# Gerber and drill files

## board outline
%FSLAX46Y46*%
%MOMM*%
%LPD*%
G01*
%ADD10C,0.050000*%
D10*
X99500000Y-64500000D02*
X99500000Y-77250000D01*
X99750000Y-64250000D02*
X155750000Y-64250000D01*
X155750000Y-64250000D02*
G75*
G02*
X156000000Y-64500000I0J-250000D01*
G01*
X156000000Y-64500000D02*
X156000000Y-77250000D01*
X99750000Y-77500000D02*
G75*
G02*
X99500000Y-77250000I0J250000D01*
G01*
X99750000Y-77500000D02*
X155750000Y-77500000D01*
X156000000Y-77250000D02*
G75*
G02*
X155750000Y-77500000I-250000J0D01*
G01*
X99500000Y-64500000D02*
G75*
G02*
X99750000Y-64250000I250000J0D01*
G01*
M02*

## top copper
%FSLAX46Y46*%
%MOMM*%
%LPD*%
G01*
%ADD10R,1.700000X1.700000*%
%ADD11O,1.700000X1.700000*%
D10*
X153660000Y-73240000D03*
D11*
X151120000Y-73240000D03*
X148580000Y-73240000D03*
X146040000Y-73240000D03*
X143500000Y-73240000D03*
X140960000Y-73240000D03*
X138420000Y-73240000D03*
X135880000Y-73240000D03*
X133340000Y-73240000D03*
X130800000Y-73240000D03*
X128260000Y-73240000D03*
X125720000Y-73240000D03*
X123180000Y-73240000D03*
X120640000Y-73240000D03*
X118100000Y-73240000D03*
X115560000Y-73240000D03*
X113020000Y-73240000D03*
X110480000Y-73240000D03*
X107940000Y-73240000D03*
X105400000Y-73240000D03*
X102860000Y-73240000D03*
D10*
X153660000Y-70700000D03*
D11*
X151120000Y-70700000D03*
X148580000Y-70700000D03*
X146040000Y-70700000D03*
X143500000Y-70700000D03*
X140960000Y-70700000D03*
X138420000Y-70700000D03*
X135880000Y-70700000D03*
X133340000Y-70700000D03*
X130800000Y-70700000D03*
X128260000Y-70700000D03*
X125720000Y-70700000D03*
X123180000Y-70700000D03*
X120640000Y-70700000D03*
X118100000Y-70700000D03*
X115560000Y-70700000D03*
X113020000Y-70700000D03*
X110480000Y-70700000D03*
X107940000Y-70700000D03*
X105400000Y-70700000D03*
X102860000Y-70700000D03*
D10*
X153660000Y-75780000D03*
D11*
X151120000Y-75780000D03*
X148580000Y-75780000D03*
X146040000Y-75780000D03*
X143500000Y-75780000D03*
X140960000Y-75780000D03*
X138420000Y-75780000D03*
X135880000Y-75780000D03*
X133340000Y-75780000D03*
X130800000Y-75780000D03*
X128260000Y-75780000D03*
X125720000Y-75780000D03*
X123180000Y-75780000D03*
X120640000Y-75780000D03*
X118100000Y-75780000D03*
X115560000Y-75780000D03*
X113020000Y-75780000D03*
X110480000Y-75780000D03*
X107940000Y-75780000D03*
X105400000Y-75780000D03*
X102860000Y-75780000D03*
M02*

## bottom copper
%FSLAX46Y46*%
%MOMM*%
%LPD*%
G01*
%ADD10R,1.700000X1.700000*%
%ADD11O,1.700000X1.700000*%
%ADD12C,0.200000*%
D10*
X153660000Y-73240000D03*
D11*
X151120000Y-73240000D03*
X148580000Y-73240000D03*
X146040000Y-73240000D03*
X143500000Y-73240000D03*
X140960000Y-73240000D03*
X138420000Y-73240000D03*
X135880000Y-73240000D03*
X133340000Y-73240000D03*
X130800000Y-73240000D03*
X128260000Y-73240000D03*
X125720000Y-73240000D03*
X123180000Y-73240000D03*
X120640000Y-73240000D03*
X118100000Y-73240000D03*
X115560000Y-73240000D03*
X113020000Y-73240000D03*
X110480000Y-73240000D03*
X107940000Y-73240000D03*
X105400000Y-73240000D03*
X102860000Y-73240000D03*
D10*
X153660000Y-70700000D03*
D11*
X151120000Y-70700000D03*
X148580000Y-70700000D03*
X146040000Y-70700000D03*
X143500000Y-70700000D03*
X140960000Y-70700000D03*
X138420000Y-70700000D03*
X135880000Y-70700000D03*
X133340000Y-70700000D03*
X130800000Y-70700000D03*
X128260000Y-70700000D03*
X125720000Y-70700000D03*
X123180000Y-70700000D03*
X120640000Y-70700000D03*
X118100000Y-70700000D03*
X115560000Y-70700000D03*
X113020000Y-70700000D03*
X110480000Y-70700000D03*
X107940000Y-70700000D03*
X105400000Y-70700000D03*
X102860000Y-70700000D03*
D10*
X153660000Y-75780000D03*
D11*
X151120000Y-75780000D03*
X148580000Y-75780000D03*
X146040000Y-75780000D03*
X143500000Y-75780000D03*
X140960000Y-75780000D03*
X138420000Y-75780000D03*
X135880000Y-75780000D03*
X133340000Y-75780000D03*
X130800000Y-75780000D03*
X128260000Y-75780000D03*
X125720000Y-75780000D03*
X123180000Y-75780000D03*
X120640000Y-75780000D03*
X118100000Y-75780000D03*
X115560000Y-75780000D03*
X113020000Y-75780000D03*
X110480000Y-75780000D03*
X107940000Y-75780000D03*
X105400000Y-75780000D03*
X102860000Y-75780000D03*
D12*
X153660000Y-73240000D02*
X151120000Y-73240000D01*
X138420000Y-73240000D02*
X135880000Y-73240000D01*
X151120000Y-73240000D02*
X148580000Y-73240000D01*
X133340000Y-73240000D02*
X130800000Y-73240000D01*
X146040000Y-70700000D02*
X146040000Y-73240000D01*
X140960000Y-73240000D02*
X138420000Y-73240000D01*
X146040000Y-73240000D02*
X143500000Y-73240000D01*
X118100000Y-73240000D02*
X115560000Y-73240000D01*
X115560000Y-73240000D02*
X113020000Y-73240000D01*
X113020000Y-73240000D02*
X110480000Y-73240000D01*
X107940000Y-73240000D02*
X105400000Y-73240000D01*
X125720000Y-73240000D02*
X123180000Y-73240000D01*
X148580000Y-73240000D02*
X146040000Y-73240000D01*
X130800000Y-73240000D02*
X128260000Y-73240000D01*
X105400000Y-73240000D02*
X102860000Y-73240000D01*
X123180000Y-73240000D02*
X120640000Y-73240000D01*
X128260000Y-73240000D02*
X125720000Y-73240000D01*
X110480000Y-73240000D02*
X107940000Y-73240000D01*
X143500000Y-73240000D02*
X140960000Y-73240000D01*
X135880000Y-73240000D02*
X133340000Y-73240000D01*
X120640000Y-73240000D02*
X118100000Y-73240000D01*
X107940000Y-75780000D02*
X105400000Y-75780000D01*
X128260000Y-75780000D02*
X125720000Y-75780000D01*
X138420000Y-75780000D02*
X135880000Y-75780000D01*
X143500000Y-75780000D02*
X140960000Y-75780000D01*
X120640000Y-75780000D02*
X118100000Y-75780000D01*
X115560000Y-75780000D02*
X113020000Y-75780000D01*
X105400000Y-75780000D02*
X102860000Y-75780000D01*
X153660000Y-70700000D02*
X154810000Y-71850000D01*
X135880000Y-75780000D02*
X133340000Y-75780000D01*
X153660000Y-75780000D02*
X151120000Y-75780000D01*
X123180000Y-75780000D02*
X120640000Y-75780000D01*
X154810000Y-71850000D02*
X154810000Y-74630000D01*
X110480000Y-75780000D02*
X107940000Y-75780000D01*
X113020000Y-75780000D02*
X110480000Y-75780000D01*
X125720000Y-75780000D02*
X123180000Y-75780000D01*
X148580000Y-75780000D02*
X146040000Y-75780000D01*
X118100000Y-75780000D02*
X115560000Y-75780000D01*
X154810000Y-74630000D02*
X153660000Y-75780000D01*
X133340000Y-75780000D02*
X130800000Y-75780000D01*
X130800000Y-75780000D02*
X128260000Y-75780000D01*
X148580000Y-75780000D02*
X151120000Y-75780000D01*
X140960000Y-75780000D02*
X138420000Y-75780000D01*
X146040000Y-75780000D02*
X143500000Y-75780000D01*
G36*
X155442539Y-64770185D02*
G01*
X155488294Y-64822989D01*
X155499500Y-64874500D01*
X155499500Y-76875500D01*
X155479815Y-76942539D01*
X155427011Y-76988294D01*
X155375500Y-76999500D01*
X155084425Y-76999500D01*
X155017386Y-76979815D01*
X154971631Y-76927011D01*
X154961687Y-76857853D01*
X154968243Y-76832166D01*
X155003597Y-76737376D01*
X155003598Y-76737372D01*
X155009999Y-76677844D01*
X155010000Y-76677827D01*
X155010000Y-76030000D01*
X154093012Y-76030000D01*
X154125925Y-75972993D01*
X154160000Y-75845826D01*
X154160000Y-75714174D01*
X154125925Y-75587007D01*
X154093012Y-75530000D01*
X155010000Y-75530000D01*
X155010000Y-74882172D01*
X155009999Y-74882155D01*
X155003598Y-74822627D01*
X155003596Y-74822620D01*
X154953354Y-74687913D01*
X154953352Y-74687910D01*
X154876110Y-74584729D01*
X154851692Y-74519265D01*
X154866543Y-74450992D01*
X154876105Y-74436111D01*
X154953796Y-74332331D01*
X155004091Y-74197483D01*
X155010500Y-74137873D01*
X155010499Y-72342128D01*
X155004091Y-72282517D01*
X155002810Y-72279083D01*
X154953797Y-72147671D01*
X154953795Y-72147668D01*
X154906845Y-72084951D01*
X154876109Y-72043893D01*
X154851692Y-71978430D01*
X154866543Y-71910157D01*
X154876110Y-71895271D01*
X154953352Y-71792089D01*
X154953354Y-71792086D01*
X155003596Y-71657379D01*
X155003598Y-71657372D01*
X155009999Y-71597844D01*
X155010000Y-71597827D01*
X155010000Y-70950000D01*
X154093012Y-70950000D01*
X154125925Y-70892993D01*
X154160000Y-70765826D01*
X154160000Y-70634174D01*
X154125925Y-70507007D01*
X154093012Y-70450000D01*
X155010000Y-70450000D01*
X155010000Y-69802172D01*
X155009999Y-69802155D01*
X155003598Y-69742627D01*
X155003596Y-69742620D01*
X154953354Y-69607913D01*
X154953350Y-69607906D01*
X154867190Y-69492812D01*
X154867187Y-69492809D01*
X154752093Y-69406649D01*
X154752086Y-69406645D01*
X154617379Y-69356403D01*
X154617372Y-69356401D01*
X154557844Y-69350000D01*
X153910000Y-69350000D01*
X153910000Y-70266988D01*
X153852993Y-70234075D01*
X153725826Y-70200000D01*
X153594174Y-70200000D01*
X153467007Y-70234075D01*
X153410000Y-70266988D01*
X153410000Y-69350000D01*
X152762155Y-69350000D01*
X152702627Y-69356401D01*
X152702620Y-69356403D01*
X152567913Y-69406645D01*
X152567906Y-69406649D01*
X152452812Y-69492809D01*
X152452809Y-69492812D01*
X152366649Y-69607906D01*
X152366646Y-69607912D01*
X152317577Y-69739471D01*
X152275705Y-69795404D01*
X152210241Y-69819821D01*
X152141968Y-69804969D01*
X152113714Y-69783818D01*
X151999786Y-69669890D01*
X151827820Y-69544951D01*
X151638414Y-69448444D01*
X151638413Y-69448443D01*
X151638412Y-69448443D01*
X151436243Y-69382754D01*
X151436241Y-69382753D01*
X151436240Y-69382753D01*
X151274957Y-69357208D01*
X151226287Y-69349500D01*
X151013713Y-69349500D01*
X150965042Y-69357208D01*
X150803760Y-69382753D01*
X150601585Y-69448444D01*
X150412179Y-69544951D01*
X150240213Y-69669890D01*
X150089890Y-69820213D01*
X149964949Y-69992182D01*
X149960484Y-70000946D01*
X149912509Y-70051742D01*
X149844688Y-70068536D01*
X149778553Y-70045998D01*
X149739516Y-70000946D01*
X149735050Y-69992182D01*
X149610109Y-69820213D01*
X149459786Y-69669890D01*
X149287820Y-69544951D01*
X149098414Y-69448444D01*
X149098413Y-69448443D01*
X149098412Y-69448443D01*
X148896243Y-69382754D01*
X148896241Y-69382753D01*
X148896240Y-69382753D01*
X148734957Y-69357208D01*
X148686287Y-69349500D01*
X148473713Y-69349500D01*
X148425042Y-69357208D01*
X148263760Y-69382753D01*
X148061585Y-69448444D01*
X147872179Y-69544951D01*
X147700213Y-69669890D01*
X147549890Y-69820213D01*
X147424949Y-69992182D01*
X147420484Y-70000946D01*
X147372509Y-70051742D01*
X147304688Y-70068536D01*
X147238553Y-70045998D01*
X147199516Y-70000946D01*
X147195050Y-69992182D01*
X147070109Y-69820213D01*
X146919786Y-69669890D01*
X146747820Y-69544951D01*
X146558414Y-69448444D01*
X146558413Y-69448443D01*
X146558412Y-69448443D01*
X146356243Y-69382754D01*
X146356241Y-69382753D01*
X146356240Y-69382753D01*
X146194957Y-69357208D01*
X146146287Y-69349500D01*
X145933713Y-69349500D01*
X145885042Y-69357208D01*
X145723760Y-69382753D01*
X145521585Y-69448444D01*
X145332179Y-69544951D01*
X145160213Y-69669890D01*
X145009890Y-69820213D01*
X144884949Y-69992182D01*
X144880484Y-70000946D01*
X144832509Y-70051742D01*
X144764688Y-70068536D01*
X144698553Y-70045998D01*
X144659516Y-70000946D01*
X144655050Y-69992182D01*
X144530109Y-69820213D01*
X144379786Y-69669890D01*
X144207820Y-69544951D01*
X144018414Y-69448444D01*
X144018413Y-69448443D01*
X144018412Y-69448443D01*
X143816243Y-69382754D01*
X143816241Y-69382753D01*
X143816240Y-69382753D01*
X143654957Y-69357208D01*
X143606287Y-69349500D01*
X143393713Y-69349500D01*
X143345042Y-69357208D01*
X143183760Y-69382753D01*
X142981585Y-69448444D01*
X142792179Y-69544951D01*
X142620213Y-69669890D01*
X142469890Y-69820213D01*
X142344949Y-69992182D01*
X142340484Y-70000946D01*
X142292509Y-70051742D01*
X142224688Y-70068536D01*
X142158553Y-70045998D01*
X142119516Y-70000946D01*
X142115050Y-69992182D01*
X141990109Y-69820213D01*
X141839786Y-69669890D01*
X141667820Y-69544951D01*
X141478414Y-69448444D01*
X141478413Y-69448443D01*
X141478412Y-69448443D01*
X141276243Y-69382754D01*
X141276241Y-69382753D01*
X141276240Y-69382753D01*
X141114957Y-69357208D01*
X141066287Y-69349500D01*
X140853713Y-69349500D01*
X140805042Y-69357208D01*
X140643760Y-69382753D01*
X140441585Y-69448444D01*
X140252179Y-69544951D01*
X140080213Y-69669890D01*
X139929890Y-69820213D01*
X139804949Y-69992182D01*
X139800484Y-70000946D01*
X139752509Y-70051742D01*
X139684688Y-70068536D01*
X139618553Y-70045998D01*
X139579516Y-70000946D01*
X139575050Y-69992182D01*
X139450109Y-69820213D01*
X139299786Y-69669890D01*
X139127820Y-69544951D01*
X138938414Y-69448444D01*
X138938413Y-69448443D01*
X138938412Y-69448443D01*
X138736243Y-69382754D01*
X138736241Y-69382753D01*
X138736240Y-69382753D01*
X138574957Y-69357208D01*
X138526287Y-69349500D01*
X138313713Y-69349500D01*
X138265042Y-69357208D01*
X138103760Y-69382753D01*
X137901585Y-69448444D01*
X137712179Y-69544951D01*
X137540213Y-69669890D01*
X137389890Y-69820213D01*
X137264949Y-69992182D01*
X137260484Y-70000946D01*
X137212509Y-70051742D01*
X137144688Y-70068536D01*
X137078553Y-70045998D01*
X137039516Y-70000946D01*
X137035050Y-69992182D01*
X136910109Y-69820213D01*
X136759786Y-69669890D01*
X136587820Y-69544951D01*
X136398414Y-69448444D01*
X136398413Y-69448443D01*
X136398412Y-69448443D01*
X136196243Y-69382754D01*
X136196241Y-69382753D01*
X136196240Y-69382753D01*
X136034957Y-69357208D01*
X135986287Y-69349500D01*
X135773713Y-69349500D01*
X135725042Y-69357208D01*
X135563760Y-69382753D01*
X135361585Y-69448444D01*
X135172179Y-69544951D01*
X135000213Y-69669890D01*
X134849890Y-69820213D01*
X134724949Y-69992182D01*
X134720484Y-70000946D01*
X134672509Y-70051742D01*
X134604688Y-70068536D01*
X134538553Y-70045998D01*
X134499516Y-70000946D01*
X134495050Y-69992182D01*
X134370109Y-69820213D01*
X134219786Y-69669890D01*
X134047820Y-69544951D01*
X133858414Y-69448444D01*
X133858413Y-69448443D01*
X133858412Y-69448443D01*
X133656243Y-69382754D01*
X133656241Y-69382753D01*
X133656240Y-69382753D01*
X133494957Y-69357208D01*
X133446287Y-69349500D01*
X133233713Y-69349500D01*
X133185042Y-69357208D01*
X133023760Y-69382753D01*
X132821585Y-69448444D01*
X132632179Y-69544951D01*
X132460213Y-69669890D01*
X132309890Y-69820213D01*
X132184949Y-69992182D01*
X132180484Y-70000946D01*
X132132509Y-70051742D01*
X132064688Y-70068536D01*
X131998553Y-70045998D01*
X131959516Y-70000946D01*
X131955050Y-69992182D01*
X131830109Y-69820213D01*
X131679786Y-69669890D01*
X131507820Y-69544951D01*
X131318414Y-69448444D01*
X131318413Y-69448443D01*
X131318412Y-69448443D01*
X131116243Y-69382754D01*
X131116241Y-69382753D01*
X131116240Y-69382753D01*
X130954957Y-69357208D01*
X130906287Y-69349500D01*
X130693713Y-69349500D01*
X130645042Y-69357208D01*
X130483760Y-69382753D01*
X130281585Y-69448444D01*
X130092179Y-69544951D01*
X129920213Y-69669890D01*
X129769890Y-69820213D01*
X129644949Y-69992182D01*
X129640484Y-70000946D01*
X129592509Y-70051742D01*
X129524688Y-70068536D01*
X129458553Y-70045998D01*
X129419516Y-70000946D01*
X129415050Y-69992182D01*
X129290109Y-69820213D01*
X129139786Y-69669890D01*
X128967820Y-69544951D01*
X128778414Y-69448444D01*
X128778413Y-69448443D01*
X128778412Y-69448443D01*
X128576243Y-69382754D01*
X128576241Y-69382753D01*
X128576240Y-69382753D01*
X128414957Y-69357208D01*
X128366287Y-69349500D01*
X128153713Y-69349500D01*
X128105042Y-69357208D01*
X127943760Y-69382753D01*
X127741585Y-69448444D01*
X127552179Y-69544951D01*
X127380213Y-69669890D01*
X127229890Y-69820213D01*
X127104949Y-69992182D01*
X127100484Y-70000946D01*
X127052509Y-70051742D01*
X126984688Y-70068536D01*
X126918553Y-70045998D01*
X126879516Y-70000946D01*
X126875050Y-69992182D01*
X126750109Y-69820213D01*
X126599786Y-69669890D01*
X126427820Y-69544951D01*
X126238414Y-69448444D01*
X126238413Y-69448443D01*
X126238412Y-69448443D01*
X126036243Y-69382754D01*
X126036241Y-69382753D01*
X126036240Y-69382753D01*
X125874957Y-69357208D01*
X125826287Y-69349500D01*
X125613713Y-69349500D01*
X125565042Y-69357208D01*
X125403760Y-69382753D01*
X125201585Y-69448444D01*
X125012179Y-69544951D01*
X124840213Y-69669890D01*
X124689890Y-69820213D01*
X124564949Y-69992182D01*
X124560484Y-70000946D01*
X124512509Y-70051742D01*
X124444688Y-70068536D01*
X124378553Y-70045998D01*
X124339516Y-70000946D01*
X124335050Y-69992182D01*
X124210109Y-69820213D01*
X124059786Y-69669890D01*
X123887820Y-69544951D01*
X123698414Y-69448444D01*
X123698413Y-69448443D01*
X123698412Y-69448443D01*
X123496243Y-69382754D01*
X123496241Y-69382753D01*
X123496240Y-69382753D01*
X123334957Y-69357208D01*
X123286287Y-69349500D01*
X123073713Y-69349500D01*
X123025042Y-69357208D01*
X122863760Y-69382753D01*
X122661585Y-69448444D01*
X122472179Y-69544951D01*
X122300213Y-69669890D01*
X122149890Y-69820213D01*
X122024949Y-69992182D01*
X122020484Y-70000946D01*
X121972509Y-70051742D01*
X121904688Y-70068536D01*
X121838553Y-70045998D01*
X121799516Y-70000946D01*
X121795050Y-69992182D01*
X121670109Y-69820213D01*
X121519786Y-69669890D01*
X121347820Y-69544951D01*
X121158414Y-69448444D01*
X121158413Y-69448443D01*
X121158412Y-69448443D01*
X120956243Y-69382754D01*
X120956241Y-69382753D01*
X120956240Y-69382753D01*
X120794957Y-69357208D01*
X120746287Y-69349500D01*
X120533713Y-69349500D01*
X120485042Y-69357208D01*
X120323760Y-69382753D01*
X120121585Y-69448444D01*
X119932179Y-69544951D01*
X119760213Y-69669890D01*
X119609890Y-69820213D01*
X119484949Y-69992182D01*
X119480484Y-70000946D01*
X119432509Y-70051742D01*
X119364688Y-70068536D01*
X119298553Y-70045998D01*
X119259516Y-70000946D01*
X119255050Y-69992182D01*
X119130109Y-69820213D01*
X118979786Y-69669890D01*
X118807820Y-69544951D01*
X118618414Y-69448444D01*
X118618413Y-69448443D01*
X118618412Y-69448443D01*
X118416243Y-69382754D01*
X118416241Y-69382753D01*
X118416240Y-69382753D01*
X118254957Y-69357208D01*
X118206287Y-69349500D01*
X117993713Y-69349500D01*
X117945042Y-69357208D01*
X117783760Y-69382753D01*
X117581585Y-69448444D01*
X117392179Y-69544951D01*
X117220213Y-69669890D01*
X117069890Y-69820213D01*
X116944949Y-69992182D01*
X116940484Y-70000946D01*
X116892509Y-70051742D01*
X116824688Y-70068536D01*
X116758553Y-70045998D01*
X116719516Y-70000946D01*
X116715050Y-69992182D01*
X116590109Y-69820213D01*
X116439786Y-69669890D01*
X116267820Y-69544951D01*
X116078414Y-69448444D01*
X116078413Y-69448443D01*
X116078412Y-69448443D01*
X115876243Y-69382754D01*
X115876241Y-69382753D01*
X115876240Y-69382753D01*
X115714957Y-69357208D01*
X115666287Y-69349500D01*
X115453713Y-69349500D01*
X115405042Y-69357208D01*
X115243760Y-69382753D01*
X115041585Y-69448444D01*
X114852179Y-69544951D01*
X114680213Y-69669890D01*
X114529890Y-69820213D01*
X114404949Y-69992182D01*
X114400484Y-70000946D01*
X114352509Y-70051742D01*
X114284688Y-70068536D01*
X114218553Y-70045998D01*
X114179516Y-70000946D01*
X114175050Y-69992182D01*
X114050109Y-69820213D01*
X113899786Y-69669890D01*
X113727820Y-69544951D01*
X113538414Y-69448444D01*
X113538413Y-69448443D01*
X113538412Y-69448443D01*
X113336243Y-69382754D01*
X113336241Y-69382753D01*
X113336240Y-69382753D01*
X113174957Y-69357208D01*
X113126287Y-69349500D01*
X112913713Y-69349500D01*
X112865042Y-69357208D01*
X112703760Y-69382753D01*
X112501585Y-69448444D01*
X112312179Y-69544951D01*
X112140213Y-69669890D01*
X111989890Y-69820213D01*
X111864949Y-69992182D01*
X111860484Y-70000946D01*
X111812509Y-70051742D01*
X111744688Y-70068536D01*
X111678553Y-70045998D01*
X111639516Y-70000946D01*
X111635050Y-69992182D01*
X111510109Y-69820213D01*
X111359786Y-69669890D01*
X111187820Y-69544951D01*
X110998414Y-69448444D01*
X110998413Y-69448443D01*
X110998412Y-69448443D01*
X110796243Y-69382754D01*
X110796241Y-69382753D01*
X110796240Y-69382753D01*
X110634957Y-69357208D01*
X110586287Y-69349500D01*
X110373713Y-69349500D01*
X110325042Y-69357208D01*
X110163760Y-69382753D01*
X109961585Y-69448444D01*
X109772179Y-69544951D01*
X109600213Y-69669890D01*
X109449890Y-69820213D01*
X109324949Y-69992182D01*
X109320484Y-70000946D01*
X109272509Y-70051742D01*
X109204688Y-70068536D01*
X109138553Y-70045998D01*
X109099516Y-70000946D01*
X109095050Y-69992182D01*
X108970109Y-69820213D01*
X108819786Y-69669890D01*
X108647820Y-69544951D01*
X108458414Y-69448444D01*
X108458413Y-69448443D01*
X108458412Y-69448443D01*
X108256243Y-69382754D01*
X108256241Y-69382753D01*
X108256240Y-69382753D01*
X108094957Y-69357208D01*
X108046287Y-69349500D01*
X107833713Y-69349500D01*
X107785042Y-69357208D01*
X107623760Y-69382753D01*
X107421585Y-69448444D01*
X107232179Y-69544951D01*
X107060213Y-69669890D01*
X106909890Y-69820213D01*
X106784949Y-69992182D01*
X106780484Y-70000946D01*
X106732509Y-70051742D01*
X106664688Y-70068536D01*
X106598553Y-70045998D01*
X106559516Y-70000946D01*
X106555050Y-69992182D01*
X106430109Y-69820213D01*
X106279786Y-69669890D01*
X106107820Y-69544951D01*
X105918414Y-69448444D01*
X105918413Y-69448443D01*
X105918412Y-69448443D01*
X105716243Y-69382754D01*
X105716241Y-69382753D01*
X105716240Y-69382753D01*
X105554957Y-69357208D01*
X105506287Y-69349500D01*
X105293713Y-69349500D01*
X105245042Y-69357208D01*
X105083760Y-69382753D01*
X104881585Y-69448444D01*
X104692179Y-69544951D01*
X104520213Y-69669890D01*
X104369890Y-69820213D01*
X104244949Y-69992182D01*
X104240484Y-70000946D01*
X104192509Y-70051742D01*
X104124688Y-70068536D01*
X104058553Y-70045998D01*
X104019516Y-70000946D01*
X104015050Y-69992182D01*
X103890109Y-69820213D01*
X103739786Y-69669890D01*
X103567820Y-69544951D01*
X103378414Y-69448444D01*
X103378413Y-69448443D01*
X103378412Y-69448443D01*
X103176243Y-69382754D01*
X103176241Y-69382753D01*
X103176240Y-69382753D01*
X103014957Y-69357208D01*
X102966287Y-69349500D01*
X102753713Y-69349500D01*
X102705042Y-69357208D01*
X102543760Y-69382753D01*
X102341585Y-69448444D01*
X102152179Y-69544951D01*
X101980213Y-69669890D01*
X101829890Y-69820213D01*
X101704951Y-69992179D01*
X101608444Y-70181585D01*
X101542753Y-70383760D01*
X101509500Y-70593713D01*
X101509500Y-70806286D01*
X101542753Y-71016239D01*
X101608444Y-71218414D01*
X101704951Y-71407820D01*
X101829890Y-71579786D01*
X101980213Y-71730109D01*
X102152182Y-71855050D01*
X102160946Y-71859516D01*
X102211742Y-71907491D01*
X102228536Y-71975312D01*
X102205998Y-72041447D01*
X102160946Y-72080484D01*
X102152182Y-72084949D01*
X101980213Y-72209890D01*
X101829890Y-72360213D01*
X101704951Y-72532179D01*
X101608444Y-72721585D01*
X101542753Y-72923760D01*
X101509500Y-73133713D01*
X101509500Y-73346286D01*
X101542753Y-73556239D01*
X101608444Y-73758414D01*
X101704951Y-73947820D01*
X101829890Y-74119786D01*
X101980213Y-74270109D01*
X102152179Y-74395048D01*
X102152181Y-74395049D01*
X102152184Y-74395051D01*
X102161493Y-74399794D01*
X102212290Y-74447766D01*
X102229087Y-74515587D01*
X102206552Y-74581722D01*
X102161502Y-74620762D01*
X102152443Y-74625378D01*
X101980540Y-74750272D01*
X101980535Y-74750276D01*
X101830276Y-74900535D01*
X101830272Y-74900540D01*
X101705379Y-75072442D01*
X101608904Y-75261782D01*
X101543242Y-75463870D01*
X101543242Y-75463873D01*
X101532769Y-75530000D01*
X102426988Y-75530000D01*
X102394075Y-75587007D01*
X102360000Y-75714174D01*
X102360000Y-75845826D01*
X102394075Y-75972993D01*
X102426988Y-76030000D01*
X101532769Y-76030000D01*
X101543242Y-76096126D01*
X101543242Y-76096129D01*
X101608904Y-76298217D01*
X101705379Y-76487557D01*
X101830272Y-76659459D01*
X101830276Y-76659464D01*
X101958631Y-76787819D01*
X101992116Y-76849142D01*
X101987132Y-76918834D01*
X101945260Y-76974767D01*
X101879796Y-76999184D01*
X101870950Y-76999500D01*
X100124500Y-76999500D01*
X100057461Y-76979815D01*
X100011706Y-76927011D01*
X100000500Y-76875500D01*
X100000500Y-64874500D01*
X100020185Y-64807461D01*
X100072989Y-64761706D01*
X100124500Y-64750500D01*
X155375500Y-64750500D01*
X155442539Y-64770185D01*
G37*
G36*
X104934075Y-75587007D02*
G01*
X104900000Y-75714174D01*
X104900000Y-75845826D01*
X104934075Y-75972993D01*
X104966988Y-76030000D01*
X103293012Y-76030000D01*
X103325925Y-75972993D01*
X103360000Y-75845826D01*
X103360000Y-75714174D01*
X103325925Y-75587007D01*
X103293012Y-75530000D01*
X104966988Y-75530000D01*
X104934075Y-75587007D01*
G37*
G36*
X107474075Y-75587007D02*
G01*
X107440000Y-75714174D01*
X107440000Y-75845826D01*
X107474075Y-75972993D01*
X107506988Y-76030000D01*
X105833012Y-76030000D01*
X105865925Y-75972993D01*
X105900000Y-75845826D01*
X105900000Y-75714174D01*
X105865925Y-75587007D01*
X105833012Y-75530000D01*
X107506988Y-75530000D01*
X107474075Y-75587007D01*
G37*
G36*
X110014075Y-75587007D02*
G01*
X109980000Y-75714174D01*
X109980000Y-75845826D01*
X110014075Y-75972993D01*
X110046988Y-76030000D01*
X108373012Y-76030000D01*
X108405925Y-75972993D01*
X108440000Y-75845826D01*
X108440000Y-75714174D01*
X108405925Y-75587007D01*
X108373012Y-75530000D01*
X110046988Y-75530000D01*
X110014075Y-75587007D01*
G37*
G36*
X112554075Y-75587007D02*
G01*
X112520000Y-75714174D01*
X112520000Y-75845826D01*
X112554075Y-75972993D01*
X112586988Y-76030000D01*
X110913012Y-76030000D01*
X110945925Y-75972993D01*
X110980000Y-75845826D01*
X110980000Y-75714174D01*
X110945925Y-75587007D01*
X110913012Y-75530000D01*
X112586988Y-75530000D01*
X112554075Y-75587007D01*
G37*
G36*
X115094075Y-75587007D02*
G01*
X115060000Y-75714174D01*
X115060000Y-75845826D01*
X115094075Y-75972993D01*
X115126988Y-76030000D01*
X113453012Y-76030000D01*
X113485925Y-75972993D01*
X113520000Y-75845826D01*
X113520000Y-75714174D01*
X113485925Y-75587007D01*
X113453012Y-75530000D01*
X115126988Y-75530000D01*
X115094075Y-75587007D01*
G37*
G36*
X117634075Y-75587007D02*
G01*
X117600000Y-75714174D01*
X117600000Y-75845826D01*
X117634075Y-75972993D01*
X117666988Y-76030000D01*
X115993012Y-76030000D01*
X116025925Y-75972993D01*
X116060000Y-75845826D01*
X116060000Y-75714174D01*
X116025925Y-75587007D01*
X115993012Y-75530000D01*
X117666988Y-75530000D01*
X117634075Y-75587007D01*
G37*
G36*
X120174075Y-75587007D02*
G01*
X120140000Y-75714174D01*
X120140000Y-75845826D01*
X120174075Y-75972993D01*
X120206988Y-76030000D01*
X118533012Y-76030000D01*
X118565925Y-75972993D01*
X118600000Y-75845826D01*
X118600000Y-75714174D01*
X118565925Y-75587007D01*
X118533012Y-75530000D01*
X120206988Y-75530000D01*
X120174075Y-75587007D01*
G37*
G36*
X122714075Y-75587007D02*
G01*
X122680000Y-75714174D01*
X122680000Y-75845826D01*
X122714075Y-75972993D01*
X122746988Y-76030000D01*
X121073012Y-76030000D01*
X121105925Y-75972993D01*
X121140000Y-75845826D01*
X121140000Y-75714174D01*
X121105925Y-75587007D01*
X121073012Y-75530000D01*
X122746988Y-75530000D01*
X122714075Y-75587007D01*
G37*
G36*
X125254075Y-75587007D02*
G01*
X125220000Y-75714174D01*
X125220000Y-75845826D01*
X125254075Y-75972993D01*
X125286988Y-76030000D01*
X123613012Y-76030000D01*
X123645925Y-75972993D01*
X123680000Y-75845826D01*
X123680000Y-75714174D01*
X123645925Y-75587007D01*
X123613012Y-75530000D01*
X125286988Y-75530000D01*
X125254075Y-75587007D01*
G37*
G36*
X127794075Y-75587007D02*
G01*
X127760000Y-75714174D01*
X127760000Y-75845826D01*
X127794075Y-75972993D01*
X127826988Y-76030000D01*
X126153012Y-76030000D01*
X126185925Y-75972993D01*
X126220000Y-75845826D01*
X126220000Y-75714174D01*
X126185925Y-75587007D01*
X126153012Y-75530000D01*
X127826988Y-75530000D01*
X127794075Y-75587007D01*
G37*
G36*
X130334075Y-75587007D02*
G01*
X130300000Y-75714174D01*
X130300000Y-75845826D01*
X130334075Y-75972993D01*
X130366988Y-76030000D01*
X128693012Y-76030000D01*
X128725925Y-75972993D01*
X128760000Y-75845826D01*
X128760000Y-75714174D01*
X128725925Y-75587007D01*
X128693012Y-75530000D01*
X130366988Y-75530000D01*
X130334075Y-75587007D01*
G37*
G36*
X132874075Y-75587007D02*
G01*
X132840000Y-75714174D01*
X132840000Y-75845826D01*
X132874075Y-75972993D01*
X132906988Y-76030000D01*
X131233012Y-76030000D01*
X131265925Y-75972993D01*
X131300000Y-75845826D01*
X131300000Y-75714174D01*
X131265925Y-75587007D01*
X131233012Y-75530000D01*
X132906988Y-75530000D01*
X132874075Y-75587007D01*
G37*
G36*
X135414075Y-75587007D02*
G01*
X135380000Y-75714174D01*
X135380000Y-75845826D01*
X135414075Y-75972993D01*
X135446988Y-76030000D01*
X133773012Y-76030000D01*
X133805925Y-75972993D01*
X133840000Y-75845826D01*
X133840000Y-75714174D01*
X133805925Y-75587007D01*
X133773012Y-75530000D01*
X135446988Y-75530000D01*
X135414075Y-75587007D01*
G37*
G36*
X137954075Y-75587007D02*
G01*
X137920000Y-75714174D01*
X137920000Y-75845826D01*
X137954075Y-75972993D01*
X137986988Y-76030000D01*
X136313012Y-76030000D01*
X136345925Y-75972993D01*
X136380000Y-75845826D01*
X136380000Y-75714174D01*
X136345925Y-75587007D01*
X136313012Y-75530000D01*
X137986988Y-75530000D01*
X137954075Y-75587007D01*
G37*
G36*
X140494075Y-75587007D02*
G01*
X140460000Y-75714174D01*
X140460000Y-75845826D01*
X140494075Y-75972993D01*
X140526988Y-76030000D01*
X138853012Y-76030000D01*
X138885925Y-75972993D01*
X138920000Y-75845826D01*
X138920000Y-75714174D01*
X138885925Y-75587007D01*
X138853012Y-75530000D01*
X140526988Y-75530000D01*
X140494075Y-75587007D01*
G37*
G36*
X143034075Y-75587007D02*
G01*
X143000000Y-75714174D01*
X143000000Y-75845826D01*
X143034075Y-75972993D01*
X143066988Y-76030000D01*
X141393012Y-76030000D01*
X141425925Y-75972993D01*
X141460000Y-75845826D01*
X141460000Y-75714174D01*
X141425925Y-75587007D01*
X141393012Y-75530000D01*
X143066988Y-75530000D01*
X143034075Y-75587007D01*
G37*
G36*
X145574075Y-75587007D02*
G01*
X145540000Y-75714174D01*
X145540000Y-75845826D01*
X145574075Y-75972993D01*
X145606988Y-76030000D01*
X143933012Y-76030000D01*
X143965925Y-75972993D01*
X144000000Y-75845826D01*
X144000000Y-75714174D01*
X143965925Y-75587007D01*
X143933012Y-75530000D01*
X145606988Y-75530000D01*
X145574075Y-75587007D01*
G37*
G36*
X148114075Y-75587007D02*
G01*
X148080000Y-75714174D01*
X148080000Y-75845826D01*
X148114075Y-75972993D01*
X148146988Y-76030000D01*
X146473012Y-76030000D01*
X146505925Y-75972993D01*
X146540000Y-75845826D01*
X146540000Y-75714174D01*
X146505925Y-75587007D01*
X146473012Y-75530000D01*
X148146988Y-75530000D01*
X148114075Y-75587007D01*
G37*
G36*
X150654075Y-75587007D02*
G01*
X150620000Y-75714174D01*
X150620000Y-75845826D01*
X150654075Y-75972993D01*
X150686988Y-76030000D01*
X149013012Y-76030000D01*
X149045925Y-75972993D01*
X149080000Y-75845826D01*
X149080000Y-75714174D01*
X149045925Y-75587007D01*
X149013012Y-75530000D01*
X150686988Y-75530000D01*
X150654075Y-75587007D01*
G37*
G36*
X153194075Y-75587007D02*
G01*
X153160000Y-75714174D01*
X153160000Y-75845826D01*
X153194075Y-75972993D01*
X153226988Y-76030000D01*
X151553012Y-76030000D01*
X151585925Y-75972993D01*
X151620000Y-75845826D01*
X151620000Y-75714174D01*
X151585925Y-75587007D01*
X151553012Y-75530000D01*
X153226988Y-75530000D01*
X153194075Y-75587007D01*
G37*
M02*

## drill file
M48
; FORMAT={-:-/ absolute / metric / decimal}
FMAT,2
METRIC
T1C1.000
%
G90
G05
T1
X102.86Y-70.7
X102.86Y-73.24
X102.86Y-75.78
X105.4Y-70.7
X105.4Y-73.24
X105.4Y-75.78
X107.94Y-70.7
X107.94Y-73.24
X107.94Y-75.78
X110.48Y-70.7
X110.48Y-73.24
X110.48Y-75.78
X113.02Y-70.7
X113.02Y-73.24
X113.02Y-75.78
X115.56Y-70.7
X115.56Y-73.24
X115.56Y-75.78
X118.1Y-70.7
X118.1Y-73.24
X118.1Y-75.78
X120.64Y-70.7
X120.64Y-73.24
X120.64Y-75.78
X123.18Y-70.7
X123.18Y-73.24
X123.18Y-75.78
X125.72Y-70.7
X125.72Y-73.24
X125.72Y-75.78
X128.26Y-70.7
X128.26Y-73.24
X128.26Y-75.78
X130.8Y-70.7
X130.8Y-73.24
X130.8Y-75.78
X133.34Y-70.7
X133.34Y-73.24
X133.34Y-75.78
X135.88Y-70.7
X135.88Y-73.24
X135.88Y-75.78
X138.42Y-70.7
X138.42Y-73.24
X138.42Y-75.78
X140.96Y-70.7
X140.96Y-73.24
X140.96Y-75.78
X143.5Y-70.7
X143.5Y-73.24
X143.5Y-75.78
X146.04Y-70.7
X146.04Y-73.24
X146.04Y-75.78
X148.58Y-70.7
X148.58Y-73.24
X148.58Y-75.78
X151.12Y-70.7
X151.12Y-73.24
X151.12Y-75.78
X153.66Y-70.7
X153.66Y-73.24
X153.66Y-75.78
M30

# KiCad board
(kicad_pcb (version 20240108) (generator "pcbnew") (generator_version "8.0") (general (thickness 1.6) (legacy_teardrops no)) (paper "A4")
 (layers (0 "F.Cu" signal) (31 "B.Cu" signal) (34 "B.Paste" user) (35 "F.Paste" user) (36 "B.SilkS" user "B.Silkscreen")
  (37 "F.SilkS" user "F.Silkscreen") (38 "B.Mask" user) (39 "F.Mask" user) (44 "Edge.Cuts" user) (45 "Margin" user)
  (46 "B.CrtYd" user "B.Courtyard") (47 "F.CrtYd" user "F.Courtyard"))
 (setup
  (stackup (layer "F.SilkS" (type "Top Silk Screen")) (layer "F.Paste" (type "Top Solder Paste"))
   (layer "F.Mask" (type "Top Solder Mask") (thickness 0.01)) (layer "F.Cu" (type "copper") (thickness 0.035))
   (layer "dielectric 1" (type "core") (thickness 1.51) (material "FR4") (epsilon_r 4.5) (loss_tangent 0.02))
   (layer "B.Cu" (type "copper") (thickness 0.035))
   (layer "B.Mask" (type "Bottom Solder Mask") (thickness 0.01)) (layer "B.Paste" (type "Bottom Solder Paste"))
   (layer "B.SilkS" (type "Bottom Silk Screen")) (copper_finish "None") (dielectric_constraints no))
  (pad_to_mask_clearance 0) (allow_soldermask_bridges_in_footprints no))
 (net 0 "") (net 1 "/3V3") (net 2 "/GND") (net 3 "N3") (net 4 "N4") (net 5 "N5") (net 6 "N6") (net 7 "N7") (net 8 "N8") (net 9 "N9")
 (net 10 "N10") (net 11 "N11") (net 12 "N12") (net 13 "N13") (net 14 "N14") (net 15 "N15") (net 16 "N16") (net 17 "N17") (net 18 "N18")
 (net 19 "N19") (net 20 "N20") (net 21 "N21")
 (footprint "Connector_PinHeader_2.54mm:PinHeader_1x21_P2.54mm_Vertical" (layer "F.Cu") (at 153.66 73.24 -90)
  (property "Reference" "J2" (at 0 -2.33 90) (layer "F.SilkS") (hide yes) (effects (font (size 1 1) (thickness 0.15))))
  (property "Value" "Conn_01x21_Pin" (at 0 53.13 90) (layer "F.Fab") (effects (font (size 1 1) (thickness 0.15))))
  (pad "1" thru_hole rect (at 0 0 270) (size 1.7 1.7) (drill 1) (layers "*.Cu" "*.Mask") (remove_unused_layers no) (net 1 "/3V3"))
  (pad "2" thru_hole oval (at 0 2.54 270) (size 1.7 1.7) (drill 1) (layers "*.Cu" "*.Mask") (remove_unused_layers no) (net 1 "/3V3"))
  (pad "3" thru_hole oval (at 0 5.08 270) (size 1.7 1.7) (drill 1) (layers "*.Cu" "*.Mask") (remove_unused_layers no) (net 1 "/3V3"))
  (pad "4" thru_hole oval (at 0 7.62 270) (size 1.7 1.7) (drill 1) (layers "*.Cu" "*.Mask") (remove_unused_layers no) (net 1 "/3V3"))
  (pad "5" thru_hole oval (at 0 10.16 270) (size 1.7 1.7) (drill 1) (layers "*.Cu" "*.Mask") (remove_unused_layers no) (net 1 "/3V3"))
  (pad "6" thru_hole oval (at 0 12.7 270) (size 1.7 1.7) (drill 1) (layers "*.Cu" "*.Mask") (remove_unused_layers no) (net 1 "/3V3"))
  (pad "7" thru_hole oval (at 0 15.24 270) (size 1.7 1.7) (drill 1) (layers "*.Cu" "*.Mask") (remove_unused_layers no) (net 1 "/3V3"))
  (pad "8" thru_hole oval (at 0 17.78 270) (size 1.7 1.7) (drill 1) (layers "*.Cu" "*.Mask") (remove_unused_layers no) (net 1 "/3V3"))
  (pad "9" thru_hole oval (at 0 20.32 270) (size 1.7 1.7) (drill 1) (layers "*.Cu" "*.Mask") (remove_unused_layers no) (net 1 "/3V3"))
  (pad "10" thru_hole oval (at 0 22.86 270) (size 1.7 1.7) (drill 1) (layers "*.Cu" "*.Mask") (remove_unused_layers no) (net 1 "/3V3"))
  (pad "11" thru_hole oval (at 0 25.4 270) (size 1.7 1.7) (drill 1) (layers "*.Cu" "*.Mask") (remove_unused_layers no) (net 1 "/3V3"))
  (pad "12" thru_hole oval (at 0 27.94 270) (size 1.7 1.7) (drill 1) (layers "*.Cu" "*.Mask") (remove_unused_layers no) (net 1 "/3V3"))
  (pad "13" thru_hole oval (at 0 30.48 270) (size 1.7 1.7) (drill 1) (layers "*.Cu" "*.Mask") (remove_unused_layers no) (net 1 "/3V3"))
  (pad "14" thru_hole oval (at 0 33.02 270) (size 1.7 1.7) (drill 1) (layers "*.Cu" "*.Mask") (remove_unused_layers no) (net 1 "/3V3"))
  (pad "15" thru_hole oval (at 0 35.56 270) (size 1.7 1.7) (drill 1) (layers "*.Cu" "*.Mask") (remove_unused_layers no) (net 1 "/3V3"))
  (pad "16" thru_hole oval (at 0 38.1 270) (size 1.7 1.7) (drill 1) (layers "*.Cu" "*.Mask") (remove_unused_layers no) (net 1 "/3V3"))
  (pad "17" thru_hole oval (at 0 40.64 270) (size 1.7 1.7) (drill 1) (layers "*.Cu" "*.Mask") (remove_unused_layers no) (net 1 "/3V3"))
  (pad "18" thru_hole oval (at 0 43.18 270) (size 1.7 1.7) (drill 1) (layers "*.Cu" "*.Mask") (remove_unused_layers no) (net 1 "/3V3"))
  (pad "19" thru_hole oval (at 0 45.72 270) (size 1.7 1.7) (drill 1) (layers "*.Cu" "*.Mask") (remove_unused_layers no) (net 1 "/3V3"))
  (pad "20" thru_hole oval (at 0 48.26 270) (size 1.7 1.7) (drill 1) (layers "*.Cu" "*.Mask") (remove_unused_layers no) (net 1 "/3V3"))
  (pad "21" thru_hole oval (at 0 50.8 270) (size 1.7 1.7) (drill 1) (layers "*.Cu" "*.Mask") (remove_unused_layers no) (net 1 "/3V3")))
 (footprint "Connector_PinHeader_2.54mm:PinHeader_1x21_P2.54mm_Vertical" (layer "F.Cu") (at 153.66 70.7 -90)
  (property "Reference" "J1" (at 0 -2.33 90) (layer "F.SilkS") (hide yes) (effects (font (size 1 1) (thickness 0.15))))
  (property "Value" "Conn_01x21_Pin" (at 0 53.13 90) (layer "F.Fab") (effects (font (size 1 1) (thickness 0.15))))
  (pad "1" thru_hole rect (at 0 0 270) (size 1.7 1.7) (drill 1) (layers "*.Cu" "*.Mask") (remove_unused_layers no) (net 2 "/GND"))
  (pad "2" thru_hole oval (at 0 2.54 270) (size 1.7 1.7) (drill 1) (layers "*.Cu" "*.Mask") (remove_unused_layers no) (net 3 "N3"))
  (pad "3" thru_hole oval (at 0 5.08 270) (size 1.7 1.7) (drill 1) (layers "*.Cu" "*.Mask") (remove_unused_layers no) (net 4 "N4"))
  (pad "4" thru_hole oval (at 0 7.62 270) (size 1.7 1.7) (drill 1) (layers "*.Cu" "*.Mask") (remove_unused_layers no) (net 1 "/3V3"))
  (pad "5" thru_hole oval (at 0 10.16 270) (size 1.7 1.7) (drill 1) (layers "*.Cu" "*.Mask") (remove_unused_layers no) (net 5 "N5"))
  (pad "6" thru_hole oval (at 0 12.7 270) (size 1.7 1.7) (drill 1) (layers "*.Cu" "*.Mask") (remove_unused_layers no) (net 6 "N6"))
  (pad "7" thru_hole oval (at 0 15.24 270) (size 1.7 1.7) (drill 1) (layers "*.Cu" "*.Mask") (remove_unused_layers no) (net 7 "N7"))
  (pad "8" thru_hole oval (at 0 17.78 270) (size 1.7 1.7) (drill 1) (layers "*.Cu" "*.Mask") (remove_unused_layers no) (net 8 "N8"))
  (pad "9" thru_hole oval (at 0 20.32 270) (size 1.7 1.7) (drill 1) (layers "*.Cu" "*.Mask") (remove_unused_layers no) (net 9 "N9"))
  (pad "10" thru_hole oval (at 0 22.86 270) (size 1.7 1.7) (drill 1) (layers "*.Cu" "*.Mask") (remove_unused_layers no) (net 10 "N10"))
  (pad "11" thru_hole oval (at 0 25.4 270) (size 1.7 1.7) (drill 1) (layers "*.Cu" "*.Mask") (remove_unused_layers no) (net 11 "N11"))
  (pad "12" thru_hole oval (at 0 27.94 270) (size 1.7 1.7) (drill 1) (layers "*.Cu" "*.Mask") (remove_unused_layers no) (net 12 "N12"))
  (pad "13" thru_hole oval (at 0 30.48 270) (size 1.7 1.7) (drill 1) (layers "*.Cu" "*.Mask") (remove_unused_layers no) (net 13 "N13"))
  (pad "14" thru_hole oval (at 0 33.02 270) (size 1.7 1.7) (drill 1) (layers "*.Cu" "*.Mask") (remove_unused_layers no) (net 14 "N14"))
  (pad "15" thru_hole oval (at 0 35.56 270) (size 1.7 1.7) (drill 1) (layers "*.Cu" "*.Mask") (remove_unused_layers no) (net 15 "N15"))
  (pad "16" thru_hole oval (at 0 38.1 270) (size 1.7 1.7) (drill 1) (layers "*.Cu" "*.Mask") (remove_unused_layers no) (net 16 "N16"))
  (pad "17" thru_hole oval (at 0 40.64 270) (size 1.7 1.7) (drill 1) (layers "*.Cu" "*.Mask") (remove_unused_layers no) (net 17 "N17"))
  (pad "18" thru_hole oval (at 0 43.18 270) (size 1.7 1.7) (drill 1) (layers "*.Cu" "*.Mask") (remove_unused_layers no) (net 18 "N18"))
  (pad "19" thru_hole oval (at 0 45.72 270) (size 1.7 1.7) (drill 1) (layers "*.Cu" "*.Mask") (remove_unused_layers no) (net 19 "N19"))
  (pad "20" thru_hole oval (at 0 48.26 270) (size 1.7 1.7) (drill 1) (layers "*.Cu" "*.Mask") (remove_unused_layers no) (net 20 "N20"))
  (pad "21" thru_hole oval (at 0 50.8 270) (size 1.7 1.7) (drill 1) (layers "*.Cu" "*.Mask") (remove_unused_layers no) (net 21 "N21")))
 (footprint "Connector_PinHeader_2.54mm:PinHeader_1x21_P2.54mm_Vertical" (layer "F.Cu") (at 153.66 75.78 -90)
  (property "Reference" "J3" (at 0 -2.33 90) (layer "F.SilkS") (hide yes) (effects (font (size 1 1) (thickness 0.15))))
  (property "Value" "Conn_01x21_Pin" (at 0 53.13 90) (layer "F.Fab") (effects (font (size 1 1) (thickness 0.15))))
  (pad "1" thru_hole rect (at 0 0 270) (size 1.7 1.7) (drill 1) (layers "*.Cu" "*.Mask") (remove_unused_layers no) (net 2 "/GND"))
  (pad "2" thru_hole oval (at 0 2.54 270) (size 1.7 1.7) (drill 1) (layers "*.Cu" "*.Mask") (remove_unused_layers no) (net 2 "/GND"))
  (pad "3" thru_hole oval (at 0 5.08 270) (size 1.7 1.7) (drill 1) (layers "*.Cu" "*.Mask") (remove_unused_layers no) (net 2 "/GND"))
  (pad "4" thru_hole oval (at 0 7.62 270) (size 1.7 1.7) (drill 1) (layers "*.Cu" "*.Mask") (remove_unused_layers no) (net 2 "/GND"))
  (pad "5" thru_hole oval (at 0 10.16 270) (size 1.7 1.7) (drill 1) (layers "*.Cu" "*.Mask") (remove_unused_layers no) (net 2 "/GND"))
  (pad "6" thru_hole oval (at 0 12.7 270) (size 1.7 1.7) (drill 1) (layers "*.Cu" "*.Mask") (remove_unused_layers no) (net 2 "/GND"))
  (pad "7" thru_hole oval (at 0 15.24 270) (size 1.7 1.7) (drill 1) (layers "*.Cu" "*.Mask") (remove_unused_layers no) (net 2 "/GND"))
  (pad "8" thru_hole oval (at 0 17.78 270) (size 1.7 1.7) (drill 1) (layers "*.Cu" "*.Mask") (remove_unused_layers no) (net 2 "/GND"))
  (pad "9" thru_hole oval (at 0 20.32 270) (size 1.7 1.7) (drill 1) (layers "*.Cu" "*.Mask") (remove_unused_layers no) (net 2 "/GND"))
  (pad "10" thru_hole oval (at 0 22.86 270) (size 1.7 1.7) (drill 1) (layers "*.Cu" "*.Mask") (remove_unused_layers no) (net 2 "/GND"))
  (pad "11" thru_hole oval (at 0 25.4 270) (size 1.7 1.7) (drill 1) (layers "*.Cu" "*.Mask") (remove_unused_layers no) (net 2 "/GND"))
  (pad "12" thru_hole oval (at 0 27.94 270) (size 1.7 1.7) (drill 1) (layers "*.Cu" "*.Mask") (remove_unused_layers no) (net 2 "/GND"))
  (pad "13" thru_hole oval (at 0 30.48 270) (size 1.7 1.7) (drill 1) (layers "*.Cu" "*.Mask") (remove_unused_layers no) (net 2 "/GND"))
  (pad "14" thru_hole oval (at 0 33.02 270) (size 1.7 1.7) (drill 1) (layers "*.Cu" "*.Mask") (remove_unused_layers no) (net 2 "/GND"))
  (pad "15" thru_hole oval (at 0 35.56 270) (size 1.7 1.7) (drill 1) (layers "*.Cu" "*.Mask") (remove_unused_layers no) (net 2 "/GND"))
  (pad "16" thru_hole oval (at 0 38.1 270) (size 1.7 1.7) (drill 1) (layers "*.Cu" "*.Mask") (remove_unused_layers no) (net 2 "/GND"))
  (pad "17" thru_hole oval (at 0 40.64 270) (size 1.7 1.7) (drill 1) (layers "*.Cu" "*.Mask") (remove_unused_layers no) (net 2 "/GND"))
  (pad "18" thru_hole oval (at 0 43.18 270) (size 1.7 1.7) (drill 1) (layers "*.Cu" "*.Mask") (remove_unused_layers no) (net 2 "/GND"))
  (pad "19" thru_hole oval (at 0 45.72 270) (size 1.7 1.7) (drill 1) (layers "*.Cu" "*.Mask") (remove_unused_layers no) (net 2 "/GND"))
  (pad "20" thru_hole oval (at 0 48.26 270) (size 1.7 1.7) (drill 1) (layers "*.Cu" "*.Mask") (remove_unused_layers no) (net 2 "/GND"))
  (pad "21" thru_hole oval (at 0 50.8 270) (size 1.7 1.7) (drill 1) (layers "*.Cu" "*.Mask") (remove_unused_layers no) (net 2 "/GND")))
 (gr_line (start 99.5 64.5) (end 99.5 77.25) (stroke (width 0.05) (type default)) (layer "Edge.Cuts"))
 (gr_line (start 99.75 64.25) (end 155.75 64.25) (stroke (width 0.05) (type default)) (layer "Edge.Cuts"))
 (gr_arc (start 155.75 64.25) (mid 155.926777 64.323223) (end 156 64.5) (stroke (width 0.05) (type default)) (layer "Edge.Cuts"))
 (gr_line (start 156 64.5) (end 156 77.25) (stroke (width 0.05) (type default)) (layer "Edge.Cuts"))
 (gr_arc (start 99.75 77.5) (mid 99.573223 77.426777) (end 99.5 77.25) (stroke (width 0.05) (type default)) (layer "Edge.Cuts"))
 (gr_line (start 99.75 77.5) (end 155.75 77.5) (stroke (width 0.05) (type default)) (layer "Edge.Cuts"))
 (gr_arc (start 156 77.25) (mid 155.926777 77.426777) (end 155.75 77.5) (stroke (width 0.05) (type default)) (layer "Edge.Cuts"))
 (gr_arc (start 99.5 64.5) (mid 99.573223 64.323223) (end 99.75 64.25) (stroke (width 0.05) (type default)) (layer "Edge.Cuts"))
 (segment (start 153.66 73.24) (end 151.12 73.24) (width 0.2) (layer "B.Cu") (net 1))
 (segment (start 138.42 73.24) (end 135.88 73.24) (width 0.2) (layer "B.Cu") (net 1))
 (segment (start 151.12 73.24) (end 148.58 73.24) (width 0.2) (layer "B.Cu") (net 1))
 (segment (start 133.34 73.24) (end 130.8 73.24) (width 0.2) (layer "B.Cu") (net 1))
 (segment (start 146.04 70.7) (end 146.04 73.24) (width 0.2) (layer "B.Cu") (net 1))
 (segment (start 140.96 73.24) (end 138.42 73.24) (width 0.2) (layer "B.Cu") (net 1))
 (segment (start 146.04 73.24) (end 143.5 73.24) (width 0.2) (layer "B.Cu") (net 1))
 (segment (start 118.1 73.24) (end 115.56 73.24) (width 0.2) (layer "B.Cu") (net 1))
 (segment (start 115.56 73.24) (end 113.02 73.24) (width 0.2) (layer "B.Cu") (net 1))
 (segment (start 113.02 73.24) (end 110.48 73.24) (width 0.2) (layer "B.Cu") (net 1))
 (segment (start 107.94 73.24) (end 105.4 73.24) (width 0.2) (layer "B.Cu") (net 1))
 (segment (start 125.72 73.24) (end 123.18 73.24) (width 0.2) (layer "B.Cu") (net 1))
 (segment (start 148.58 73.24) (end 146.04 73.24) (width 0.2) (layer "B.Cu") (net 1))
 (segment (start 130.8 73.24) (end 128.26 73.24) (width 0.2) (layer "B.Cu") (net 1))
 (segment (start 105.4 73.24) (end 102.86 73.24) (width 0.2) (layer "B.Cu") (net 1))
 (segment (start 123.18 73.24) (end 120.64 73.24) (width 0.2) (layer "B.Cu") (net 1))
 (segment (start 128.26 73.24) (end 125.72 73.24) (width 0.2) (layer "B.Cu") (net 1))
 (segment (start 110.48 73.24) (end 107.94 73.24) (width 0.2) (layer "B.Cu") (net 1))
 (segment (start 143.5 73.24) (end 140.96 73.24) (width 0.2) (layer "B.Cu") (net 1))
 (segment (start 135.88 73.24) (end 133.34 73.24) (width 0.2) (layer "B.Cu") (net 1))
 (segment (start 120.64 73.24) (end 118.1 73.24) (width 0.2) (layer "B.Cu") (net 1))
 (segment (start 107.94 75.78) (end 105.4 75.78) (width 0.2) (layer "B.Cu") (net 2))
 (segment (start 128.26 75.78) (end 125.72 75.78) (width 0.2) (layer "B.Cu") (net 2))
 (segment (start 138.42 75.78) (end 135.88 75.78) (width 0.2) (layer "B.Cu") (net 2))
 (segment (start 143.5 75.78) (end 140.96 75.78) (width 0.2) (layer "B.Cu") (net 2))
 (segment (start 120.64 75.78) (end 118.1 75.78) (width 0.2) (layer "B.Cu") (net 2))
 (segment (start 115.56 75.78) (end 113.02 75.78) (width 0.2) (layer "B.Cu") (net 2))
 (segment (start 105.4 75.78) (end 102.86 75.78) (width 0.2) (layer "B.Cu") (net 2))
 (segment (start 153.66 70.7) (end 154.81 71.85) (width 0.2) (layer "B.Cu") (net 2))
 (segment (start 135.88 75.78) (end 133.34 75.78) (width 0.2) (layer "B.Cu") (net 2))
 (segment (start 153.66 75.78) (end 151.12 75.78) (width 0.2) (layer "B.Cu") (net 2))
 (segment (start 123.18 75.78) (end 120.64 75.78) (width 0.2) (layer "B.Cu") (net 2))
 (segment (start 154.81 71.85) (end 154.81 74.63) (width 0.2) (layer "B.Cu") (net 2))
 (segment (start 110.48 75.78) (end 107.94 75.78) (width 0.2) (layer "B.Cu") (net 2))
 (segment (start 113.02 75.78) (end 110.48 75.78) (width 0.2) (layer "B.Cu") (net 2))
 (segment (start 125.72 75.78) (end 123.18 75.78) (width 0.2) (layer "B.Cu") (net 2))
 (segment (start 148.58 75.78) (end 146.04 75.78) (width 0.2) (layer "B.Cu") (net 2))
 (segment (start 118.1 75.78) (end 115.56 75.78) (width 0.2) (layer "B.Cu") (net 2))
 (segment (start 154.81 74.63) (end 153.66 75.78) (width 0.2) (layer "B.Cu") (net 2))
 (segment (start 133.34 75.78) (end 130.8 75.78) (width 0.2) (layer "B.Cu") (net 2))
 (segment (start 130.8 75.78) (end 128.26 75.78) (width 0.2) (layer "B.Cu") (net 2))
 (segment (start 148.58 75.78) (end 151.12 75.78) (width 0.2) (layer "B.Cu") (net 2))
 (segment (start 140.96 75.78) (end 138.42 75.78) (width 0.2) (layer "B.Cu") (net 2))
 (segment (start 146.04 75.78) (end 143.5 75.78) (width 0.2) (layer "B.Cu") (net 2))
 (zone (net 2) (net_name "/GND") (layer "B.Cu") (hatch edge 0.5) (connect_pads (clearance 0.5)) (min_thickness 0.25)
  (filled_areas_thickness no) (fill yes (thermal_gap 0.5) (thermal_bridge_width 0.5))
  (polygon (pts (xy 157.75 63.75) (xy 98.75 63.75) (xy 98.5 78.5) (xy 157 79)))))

